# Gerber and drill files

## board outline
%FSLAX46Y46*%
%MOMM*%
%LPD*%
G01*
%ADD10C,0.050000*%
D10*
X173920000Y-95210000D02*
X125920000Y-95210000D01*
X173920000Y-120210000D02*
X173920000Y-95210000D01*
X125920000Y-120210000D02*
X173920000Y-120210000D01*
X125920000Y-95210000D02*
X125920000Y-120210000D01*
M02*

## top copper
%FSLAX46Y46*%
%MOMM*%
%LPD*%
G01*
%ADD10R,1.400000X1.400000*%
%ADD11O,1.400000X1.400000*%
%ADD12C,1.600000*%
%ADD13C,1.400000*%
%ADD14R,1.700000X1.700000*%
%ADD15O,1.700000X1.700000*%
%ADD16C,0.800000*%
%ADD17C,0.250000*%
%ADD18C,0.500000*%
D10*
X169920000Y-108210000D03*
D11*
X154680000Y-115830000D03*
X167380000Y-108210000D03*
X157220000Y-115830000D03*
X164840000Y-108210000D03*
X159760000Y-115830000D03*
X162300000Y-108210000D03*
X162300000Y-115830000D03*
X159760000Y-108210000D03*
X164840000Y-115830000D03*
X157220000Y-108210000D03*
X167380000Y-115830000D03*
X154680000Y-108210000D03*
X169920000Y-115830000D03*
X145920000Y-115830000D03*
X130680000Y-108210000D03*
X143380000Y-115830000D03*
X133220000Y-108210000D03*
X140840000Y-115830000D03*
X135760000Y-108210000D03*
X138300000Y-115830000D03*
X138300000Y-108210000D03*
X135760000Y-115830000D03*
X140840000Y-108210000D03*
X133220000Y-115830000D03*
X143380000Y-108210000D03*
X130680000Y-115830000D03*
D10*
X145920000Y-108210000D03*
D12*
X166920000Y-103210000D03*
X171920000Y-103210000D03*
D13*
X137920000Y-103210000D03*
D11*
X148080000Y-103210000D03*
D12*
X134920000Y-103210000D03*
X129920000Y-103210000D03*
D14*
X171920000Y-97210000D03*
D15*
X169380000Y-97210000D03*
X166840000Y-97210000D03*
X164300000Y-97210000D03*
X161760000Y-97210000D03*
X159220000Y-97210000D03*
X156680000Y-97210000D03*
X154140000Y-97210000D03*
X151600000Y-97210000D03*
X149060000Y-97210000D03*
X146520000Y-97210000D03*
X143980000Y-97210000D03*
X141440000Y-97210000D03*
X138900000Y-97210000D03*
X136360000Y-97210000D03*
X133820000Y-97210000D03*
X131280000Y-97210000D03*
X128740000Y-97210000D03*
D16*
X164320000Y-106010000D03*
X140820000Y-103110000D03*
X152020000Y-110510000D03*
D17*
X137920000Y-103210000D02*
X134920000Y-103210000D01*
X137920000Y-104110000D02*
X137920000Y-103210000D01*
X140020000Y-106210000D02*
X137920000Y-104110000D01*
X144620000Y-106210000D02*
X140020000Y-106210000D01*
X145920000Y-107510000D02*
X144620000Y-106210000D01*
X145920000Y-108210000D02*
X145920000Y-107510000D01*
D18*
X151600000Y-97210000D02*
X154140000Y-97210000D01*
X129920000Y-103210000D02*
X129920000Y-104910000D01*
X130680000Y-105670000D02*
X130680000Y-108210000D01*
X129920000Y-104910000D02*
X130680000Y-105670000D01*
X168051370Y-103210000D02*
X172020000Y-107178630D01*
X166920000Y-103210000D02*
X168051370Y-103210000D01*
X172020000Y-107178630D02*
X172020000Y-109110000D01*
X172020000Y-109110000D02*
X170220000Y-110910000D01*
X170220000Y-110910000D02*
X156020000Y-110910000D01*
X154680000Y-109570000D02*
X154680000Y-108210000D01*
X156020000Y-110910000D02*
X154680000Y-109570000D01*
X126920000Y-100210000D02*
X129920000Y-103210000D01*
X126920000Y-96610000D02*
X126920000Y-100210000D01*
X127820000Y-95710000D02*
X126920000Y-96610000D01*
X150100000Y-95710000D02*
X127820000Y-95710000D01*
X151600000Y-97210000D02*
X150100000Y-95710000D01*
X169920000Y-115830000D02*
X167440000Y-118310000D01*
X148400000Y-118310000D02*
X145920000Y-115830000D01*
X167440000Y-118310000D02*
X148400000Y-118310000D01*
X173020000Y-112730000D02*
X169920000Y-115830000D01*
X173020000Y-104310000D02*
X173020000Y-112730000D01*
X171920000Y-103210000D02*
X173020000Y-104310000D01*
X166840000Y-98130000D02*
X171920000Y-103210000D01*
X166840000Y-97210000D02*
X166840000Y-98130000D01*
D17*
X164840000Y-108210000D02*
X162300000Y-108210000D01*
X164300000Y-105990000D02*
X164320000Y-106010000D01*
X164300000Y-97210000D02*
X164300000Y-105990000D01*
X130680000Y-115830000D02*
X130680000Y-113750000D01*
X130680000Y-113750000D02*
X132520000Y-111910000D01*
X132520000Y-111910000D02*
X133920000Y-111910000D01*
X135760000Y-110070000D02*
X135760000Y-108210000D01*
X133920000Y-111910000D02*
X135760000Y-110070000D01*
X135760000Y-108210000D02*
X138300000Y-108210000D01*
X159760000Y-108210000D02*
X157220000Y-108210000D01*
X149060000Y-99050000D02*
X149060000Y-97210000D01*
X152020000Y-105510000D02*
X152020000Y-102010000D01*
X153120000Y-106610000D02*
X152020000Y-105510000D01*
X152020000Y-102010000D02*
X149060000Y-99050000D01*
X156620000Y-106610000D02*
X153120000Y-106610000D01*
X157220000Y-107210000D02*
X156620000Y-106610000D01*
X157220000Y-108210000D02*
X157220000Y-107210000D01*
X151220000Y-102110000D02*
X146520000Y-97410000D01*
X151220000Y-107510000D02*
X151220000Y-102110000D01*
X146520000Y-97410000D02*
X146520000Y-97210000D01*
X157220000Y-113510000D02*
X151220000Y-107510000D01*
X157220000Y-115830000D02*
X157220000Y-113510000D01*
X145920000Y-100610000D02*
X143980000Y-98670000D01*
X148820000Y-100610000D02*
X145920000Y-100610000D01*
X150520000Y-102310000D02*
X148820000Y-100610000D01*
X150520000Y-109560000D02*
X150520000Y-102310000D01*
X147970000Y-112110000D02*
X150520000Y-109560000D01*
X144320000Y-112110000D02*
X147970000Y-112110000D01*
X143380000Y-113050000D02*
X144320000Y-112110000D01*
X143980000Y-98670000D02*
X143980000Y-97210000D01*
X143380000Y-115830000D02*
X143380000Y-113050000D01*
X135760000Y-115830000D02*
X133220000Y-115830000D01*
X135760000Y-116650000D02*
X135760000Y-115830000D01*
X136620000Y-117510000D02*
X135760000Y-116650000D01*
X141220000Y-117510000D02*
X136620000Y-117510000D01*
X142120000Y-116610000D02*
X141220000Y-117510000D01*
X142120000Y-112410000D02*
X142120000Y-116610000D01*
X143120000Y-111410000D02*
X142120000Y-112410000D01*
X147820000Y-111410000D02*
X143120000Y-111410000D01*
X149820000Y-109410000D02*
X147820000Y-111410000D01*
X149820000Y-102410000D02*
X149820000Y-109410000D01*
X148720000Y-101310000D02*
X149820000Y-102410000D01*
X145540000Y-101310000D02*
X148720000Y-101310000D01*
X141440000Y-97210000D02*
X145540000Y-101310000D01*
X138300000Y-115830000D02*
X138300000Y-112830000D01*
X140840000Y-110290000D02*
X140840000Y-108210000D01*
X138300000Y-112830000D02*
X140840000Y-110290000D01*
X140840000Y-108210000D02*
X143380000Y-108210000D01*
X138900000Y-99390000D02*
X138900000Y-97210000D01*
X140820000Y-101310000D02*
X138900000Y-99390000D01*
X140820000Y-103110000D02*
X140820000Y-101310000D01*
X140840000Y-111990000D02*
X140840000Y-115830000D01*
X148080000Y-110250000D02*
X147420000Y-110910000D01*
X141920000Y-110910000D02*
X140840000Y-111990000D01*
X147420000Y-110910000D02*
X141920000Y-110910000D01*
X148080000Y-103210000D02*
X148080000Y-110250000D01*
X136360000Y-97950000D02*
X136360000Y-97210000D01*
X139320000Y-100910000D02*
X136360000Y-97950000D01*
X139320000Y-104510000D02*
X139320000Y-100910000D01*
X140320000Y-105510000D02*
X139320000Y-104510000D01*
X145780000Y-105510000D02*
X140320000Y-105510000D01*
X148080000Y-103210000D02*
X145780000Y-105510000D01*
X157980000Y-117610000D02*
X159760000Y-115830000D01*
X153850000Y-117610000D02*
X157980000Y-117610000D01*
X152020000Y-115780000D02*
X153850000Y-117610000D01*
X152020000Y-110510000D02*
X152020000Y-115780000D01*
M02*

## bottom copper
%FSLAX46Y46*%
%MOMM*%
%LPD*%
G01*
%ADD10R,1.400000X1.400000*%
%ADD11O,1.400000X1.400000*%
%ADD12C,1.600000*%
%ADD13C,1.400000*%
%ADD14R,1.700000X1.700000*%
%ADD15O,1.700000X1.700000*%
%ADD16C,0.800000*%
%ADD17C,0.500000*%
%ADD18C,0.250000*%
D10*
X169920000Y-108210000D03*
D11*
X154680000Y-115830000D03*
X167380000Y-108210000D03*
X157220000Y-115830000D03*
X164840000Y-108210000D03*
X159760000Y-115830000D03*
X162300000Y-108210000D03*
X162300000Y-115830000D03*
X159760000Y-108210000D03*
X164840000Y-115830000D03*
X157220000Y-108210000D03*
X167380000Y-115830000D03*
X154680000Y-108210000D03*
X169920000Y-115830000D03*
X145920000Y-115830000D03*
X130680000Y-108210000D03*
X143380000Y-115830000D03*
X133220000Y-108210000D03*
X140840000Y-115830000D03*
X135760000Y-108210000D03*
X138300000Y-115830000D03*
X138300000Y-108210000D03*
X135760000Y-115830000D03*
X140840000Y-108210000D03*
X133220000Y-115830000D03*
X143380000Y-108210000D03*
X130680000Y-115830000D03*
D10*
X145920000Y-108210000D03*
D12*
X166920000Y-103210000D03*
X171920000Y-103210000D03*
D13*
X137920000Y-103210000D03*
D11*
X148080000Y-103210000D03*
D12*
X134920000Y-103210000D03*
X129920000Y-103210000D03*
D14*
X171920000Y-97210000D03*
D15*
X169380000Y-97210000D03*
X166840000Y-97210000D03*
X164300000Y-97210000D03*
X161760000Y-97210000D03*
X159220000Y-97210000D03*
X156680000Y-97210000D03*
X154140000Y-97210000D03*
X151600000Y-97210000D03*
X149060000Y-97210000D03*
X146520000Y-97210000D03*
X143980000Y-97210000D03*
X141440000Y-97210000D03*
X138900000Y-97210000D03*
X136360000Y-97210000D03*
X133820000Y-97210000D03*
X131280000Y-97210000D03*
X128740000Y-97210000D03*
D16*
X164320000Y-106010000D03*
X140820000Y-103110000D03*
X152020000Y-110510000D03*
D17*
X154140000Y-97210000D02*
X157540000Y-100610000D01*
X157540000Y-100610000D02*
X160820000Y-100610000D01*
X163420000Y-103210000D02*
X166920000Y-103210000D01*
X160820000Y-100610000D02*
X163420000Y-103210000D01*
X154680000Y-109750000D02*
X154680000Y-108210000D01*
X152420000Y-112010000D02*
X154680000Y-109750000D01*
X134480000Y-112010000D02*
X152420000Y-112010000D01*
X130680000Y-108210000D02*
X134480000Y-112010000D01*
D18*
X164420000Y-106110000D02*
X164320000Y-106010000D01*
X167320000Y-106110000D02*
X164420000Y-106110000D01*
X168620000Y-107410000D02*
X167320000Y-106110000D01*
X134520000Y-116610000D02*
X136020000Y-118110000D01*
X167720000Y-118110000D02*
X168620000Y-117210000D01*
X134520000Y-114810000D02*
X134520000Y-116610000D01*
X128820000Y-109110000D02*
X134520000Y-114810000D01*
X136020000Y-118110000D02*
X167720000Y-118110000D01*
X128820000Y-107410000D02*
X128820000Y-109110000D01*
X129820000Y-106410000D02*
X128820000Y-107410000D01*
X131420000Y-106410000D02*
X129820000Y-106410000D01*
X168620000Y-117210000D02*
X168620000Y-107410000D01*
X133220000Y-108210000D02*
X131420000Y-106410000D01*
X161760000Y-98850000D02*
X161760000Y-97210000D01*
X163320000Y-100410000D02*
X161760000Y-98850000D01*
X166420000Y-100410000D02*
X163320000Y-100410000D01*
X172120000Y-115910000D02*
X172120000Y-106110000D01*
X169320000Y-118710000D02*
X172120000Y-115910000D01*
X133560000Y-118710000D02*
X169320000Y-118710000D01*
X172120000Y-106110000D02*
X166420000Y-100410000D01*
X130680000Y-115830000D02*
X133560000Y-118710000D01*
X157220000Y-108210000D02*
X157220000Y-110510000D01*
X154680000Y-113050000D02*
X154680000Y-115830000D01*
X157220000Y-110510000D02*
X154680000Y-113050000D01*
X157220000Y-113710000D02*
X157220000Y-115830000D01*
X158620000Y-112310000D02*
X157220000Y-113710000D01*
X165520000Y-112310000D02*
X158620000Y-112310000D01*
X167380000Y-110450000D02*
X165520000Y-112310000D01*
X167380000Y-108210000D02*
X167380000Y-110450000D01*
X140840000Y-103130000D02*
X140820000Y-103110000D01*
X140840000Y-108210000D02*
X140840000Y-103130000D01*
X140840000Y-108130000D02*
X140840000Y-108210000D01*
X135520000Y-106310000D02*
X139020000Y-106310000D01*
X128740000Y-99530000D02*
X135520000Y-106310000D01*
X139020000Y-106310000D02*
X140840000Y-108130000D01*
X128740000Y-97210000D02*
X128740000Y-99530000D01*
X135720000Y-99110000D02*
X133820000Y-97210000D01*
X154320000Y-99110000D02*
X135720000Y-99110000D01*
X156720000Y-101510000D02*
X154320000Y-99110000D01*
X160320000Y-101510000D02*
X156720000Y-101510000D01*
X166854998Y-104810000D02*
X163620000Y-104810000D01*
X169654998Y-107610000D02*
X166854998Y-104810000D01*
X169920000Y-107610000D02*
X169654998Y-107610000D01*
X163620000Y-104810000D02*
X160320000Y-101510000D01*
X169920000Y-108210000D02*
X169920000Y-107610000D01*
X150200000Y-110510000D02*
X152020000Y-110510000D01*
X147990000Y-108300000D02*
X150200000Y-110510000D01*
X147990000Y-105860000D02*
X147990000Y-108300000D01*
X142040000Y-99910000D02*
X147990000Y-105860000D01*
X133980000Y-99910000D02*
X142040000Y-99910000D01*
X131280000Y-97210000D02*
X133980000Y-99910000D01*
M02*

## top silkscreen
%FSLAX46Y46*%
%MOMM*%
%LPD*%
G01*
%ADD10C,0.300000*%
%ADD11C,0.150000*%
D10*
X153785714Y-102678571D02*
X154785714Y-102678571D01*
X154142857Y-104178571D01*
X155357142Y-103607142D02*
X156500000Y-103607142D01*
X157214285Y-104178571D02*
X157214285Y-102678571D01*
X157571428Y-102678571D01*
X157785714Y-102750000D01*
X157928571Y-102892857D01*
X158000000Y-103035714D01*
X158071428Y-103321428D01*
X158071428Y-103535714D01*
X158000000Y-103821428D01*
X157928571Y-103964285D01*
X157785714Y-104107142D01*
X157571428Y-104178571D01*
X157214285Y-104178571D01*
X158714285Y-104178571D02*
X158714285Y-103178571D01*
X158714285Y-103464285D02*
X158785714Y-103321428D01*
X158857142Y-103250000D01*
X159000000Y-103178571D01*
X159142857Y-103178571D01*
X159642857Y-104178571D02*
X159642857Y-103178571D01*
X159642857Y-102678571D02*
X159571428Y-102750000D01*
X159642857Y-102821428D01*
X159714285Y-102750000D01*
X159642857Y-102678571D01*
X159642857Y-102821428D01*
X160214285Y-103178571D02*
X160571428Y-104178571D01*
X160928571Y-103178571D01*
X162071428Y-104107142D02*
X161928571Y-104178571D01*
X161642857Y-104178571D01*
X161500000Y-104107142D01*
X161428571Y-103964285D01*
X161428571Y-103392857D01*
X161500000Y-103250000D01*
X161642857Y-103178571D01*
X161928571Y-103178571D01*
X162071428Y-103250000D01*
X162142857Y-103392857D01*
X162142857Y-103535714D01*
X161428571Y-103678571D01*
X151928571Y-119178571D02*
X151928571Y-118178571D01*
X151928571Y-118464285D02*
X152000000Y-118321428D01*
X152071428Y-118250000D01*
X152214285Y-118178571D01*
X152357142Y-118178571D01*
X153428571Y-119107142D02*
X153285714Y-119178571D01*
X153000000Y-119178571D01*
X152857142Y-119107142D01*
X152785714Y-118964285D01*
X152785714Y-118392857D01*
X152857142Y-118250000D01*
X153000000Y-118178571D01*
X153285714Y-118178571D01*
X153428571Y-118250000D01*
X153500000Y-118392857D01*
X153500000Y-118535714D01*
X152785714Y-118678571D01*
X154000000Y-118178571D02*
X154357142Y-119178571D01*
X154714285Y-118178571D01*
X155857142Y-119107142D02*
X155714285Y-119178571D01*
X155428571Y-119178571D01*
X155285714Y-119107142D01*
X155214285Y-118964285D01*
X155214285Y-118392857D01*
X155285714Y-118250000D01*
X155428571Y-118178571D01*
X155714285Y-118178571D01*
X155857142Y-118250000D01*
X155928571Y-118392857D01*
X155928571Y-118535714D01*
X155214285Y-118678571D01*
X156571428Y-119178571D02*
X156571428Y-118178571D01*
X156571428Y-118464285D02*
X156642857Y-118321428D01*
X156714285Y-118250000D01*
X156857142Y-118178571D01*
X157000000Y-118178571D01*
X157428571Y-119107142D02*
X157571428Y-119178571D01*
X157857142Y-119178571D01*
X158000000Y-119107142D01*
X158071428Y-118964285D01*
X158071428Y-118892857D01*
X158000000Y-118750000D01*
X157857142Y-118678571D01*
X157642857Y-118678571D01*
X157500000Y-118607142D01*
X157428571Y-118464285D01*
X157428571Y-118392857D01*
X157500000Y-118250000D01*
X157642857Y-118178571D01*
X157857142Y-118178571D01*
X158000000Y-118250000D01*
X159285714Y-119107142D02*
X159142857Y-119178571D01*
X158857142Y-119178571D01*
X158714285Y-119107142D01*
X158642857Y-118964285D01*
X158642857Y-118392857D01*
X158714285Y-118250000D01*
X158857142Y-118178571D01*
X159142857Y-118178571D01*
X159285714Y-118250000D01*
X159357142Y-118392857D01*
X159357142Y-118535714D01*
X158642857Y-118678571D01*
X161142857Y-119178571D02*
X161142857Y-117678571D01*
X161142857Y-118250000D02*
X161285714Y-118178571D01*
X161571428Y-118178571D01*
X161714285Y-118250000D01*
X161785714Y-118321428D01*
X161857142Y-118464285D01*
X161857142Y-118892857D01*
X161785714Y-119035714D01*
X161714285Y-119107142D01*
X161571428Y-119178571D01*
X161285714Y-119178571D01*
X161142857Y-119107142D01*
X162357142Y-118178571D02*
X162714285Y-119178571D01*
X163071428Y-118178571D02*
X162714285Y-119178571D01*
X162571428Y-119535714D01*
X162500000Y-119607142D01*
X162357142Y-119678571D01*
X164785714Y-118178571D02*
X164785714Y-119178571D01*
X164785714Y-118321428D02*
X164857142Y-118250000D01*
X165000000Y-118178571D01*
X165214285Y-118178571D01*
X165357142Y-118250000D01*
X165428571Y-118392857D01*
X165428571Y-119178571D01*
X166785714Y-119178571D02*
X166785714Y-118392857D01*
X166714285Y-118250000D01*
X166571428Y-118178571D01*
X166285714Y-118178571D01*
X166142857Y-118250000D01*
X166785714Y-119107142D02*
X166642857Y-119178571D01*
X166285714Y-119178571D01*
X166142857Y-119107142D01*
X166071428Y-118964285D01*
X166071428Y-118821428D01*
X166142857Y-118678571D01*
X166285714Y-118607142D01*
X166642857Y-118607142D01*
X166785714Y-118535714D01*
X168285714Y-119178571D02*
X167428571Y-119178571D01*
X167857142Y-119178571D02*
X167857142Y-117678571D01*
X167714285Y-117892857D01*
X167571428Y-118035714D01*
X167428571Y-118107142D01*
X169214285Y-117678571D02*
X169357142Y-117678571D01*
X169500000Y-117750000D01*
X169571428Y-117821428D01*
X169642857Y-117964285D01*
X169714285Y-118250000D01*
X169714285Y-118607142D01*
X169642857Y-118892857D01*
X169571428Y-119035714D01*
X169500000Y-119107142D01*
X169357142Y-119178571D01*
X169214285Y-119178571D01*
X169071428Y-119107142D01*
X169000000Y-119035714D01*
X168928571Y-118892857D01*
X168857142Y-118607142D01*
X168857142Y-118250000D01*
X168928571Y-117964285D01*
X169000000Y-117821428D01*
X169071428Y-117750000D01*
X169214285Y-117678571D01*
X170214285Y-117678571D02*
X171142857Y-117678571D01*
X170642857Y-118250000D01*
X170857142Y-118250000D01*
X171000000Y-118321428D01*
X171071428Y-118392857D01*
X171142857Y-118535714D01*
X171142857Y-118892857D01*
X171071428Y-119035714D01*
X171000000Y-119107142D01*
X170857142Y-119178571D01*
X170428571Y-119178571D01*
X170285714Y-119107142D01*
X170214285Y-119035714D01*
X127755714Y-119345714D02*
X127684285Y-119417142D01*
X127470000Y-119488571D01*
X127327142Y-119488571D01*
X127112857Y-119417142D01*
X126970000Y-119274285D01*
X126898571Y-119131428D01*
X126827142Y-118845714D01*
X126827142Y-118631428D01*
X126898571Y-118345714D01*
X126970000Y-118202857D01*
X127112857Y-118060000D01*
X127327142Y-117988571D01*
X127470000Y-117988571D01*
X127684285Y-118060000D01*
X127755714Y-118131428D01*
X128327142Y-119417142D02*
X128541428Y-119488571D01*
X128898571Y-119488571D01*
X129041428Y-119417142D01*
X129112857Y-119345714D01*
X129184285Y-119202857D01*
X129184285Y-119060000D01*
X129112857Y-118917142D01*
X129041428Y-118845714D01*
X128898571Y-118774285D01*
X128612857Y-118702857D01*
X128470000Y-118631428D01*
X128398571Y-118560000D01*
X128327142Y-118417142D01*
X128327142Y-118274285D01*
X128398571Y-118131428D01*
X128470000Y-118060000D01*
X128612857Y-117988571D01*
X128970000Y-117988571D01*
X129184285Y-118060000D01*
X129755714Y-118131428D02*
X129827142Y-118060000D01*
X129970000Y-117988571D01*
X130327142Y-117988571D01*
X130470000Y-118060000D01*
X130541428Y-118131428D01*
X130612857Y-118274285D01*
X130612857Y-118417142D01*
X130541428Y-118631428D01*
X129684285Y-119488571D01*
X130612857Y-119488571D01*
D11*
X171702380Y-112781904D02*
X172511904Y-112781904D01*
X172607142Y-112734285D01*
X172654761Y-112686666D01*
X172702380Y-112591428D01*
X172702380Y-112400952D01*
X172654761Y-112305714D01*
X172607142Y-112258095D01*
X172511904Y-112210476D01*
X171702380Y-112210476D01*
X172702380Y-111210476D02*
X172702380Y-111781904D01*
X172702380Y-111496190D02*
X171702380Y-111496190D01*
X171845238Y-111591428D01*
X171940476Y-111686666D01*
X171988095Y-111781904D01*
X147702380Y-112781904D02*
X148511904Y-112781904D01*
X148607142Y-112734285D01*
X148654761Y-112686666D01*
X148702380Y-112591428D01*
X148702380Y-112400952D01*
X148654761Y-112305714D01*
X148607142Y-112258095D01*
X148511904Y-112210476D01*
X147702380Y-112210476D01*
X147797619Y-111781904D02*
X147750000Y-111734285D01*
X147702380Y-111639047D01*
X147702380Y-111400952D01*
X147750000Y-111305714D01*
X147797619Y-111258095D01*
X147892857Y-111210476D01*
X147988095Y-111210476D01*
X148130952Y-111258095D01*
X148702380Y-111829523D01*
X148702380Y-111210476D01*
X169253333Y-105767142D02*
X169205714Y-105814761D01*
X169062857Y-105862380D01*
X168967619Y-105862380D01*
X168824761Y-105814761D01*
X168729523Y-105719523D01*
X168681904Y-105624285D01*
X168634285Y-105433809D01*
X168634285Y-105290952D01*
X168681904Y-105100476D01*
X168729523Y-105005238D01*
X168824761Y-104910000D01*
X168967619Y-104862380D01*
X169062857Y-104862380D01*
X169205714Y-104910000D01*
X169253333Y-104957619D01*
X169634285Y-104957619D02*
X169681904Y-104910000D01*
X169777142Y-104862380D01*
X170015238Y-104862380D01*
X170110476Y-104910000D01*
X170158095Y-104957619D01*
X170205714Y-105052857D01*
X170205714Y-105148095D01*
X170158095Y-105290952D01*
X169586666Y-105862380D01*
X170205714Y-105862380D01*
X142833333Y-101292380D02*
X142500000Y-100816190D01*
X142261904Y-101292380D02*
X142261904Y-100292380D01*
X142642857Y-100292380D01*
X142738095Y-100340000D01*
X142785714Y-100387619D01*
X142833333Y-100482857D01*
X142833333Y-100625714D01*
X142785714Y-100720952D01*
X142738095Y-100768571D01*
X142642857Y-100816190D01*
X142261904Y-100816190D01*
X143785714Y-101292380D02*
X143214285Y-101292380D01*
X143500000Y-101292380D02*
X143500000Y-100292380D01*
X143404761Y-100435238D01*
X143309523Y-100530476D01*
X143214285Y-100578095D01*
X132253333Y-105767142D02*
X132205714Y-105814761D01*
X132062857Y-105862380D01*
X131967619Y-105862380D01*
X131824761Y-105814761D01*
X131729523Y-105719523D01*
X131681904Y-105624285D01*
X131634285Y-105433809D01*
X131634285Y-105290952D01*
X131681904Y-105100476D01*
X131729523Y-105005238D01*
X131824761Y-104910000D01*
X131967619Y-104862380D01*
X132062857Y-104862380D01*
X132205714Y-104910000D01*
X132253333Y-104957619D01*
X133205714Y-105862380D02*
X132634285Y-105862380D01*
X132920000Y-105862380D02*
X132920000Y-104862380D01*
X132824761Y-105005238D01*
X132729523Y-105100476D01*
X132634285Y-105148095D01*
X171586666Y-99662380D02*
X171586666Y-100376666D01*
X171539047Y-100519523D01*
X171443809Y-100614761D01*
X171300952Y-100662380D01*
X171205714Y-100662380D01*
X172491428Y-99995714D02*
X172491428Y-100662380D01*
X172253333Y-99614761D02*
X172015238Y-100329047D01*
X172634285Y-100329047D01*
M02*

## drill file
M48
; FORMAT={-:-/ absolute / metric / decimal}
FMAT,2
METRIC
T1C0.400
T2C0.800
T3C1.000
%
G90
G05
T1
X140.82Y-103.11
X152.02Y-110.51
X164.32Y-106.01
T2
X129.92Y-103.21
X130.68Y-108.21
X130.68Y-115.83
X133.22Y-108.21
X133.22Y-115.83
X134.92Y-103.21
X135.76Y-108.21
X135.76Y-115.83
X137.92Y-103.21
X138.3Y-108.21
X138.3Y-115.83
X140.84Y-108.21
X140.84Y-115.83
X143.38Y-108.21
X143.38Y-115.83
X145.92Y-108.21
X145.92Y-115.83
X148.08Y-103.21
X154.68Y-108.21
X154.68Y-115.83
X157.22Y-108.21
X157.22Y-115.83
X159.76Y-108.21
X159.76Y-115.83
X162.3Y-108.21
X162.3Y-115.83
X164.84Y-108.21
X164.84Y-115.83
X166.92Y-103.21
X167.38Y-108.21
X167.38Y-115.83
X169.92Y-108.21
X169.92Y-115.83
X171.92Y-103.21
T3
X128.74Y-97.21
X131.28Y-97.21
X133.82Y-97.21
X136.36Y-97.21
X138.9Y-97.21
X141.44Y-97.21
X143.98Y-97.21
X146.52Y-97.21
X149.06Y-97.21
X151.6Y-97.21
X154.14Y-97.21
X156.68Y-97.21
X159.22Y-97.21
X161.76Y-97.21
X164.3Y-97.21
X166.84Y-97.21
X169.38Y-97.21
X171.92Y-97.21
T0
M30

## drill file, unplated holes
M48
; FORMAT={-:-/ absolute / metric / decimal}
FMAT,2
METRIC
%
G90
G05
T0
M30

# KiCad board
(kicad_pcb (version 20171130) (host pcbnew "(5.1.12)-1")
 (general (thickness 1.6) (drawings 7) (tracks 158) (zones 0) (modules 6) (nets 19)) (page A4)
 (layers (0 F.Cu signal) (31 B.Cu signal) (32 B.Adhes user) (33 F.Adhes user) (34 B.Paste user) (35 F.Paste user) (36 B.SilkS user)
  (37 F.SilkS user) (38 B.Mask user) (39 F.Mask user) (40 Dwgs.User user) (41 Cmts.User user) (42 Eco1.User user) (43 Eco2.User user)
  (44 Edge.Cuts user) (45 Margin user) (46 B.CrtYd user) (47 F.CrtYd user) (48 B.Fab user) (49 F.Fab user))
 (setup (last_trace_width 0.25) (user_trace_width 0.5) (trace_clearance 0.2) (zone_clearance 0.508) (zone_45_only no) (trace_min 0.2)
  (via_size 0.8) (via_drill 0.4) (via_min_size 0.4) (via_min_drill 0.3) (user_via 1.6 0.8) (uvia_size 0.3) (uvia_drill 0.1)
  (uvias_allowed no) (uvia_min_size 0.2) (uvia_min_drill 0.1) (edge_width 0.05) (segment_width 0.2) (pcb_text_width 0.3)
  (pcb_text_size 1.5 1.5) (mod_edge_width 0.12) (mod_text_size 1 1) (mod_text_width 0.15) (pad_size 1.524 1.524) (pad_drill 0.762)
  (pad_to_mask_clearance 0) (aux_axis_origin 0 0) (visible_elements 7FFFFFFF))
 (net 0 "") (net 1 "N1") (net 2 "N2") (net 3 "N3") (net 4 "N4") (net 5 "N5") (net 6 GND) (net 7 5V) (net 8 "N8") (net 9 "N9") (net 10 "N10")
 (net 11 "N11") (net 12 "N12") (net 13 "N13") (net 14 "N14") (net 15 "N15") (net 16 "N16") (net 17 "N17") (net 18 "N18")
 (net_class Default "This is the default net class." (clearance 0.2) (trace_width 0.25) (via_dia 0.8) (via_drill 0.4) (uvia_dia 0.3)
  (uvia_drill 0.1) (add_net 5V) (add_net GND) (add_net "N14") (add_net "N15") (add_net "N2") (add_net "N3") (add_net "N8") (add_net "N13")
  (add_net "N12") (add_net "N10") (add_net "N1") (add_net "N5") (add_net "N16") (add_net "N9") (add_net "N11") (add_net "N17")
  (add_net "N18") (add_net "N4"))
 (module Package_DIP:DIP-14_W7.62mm (layer F.Cu) (at 169.92 108.21 270)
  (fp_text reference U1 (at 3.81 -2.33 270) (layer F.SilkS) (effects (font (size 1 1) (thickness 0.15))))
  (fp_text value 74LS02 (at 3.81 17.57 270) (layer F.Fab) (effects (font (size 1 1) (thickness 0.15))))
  (pad 1 thru_hole rect (at 0 0 270) (size 1.4 1.4) (drill 0.8) (layers *.Cu *.Mask) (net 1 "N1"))
  (pad 8 thru_hole oval (at 7.62 15.24 270) (size 1.4 1.4) (drill 0.8) (layers *.Cu *.Mask) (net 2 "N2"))
  (pad 2 thru_hole oval (at 0 2.54 270) (size 1.4 1.4) (drill 0.8) (layers *.Cu *.Mask) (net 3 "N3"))
  (pad 9 thru_hole oval (at 7.62 12.7 270) (size 1.4 1.4) (drill 0.8) (layers *.Cu *.Mask) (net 3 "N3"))
  (pad 3 thru_hole oval (at 0 5.08 270) (size 1.4 1.4) (drill 0.8) (layers *.Cu *.Mask) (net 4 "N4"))
  (pad 10 thru_hole oval (at 7.62 10.16 270) (size 1.4 1.4) (drill 0.8) (layers *.Cu *.Mask) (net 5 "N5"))
  (pad 4 thru_hole oval (at 0 7.62 270) (size 1.4 1.4) (drill 0.8) (layers *.Cu *.Mask) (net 4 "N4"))
  (pad 11 thru_hole oval (at 7.62 7.62 270) (size 1.4 1.4) (drill 0.8) (layers *.Cu *.Mask))
  (pad 5 thru_hole oval (at 0 10.16 270) (size 1.4 1.4) (drill 0.8) (layers *.Cu *.Mask) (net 2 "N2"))
  (pad 12 thru_hole oval (at 7.62 5.08 270) (size 1.4 1.4) (drill 0.8) (layers *.Cu *.Mask))
  (pad 6 thru_hole oval (at 0 12.7 270) (size 1.4 1.4) (drill 0.8) (layers *.Cu *.Mask) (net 2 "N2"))
  (pad 13 thru_hole oval (at 7.62 2.54 270) (size 1.4 1.4) (drill 0.8) (layers *.Cu *.Mask))
  (pad 7 thru_hole oval (at 0 15.24 270) (size 1.4 1.4) (drill 0.8) (layers *.Cu *.Mask) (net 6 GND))
  (pad 14 thru_hole oval (at 7.62 0 270) (size 1.4 1.4) (drill 0.8) (layers *.Cu *.Mask) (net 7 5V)))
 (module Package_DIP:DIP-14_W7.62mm (layer F.Cu) (at 145.92 108.21 270)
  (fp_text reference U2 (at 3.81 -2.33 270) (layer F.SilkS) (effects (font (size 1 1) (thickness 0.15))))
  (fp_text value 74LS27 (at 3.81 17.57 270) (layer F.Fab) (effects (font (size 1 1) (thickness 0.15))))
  (pad 14 thru_hole oval (at 7.62 0 270) (size 1.4 1.4) (drill 0.8) (layers *.Cu *.Mask) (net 7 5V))
  (pad 7 thru_hole oval (at 0 15.24 270) (size 1.4 1.4) (drill 0.8) (layers *.Cu *.Mask) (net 6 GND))
  (pad 13 thru_hole oval (at 7.62 2.54 270) (size 1.4 1.4) (drill 0.8) (layers *.Cu *.Mask) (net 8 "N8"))
  (pad 6 thru_hole oval (at 0 12.7 270) (size 1.4 1.4) (drill 0.8) (layers *.Cu *.Mask) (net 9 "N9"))
  (pad 12 thru_hole oval (at 7.62 5.08 270) (size 1.4 1.4) (drill 0.8) (layers *.Cu *.Mask) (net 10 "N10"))
  (pad 5 thru_hole oval (at 0 10.16 270) (size 1.4 1.4) (drill 0.8) (layers *.Cu *.Mask) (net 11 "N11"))
  (pad 11 thru_hole oval (at 7.62 7.62 270) (size 1.4 1.4) (drill 0.8) (layers *.Cu *.Mask) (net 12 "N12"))
  (pad 4 thru_hole oval (at 0 7.62 270) (size 1.4 1.4) (drill 0.8) (layers *.Cu *.Mask) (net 11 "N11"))
  (pad 10 thru_hole oval (at 7.62 10.16 270) (size 1.4 1.4) (drill 0.8) (layers *.Cu *.Mask) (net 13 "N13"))
  (pad 3 thru_hole oval (at 0 5.08 270) (size 1.4 1.4) (drill 0.8) (layers *.Cu *.Mask) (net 12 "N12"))
  (pad 9 thru_hole oval (at 7.62 12.7 270) (size 1.4 1.4) (drill 0.8) (layers *.Cu *.Mask) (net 13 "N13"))
  (pad 2 thru_hole oval (at 0 2.54 270) (size 1.4 1.4) (drill 0.8) (layers *.Cu *.Mask) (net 12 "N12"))
  (pad 8 thru_hole oval (at 7.62 15.24 270) (size 1.4 1.4) (drill 0.8) (layers *.Cu *.Mask) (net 11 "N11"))
  (pad 1 thru_hole rect (at 0 0 270) (size 1.4 1.4) (drill 0.8) (layers *.Cu *.Mask) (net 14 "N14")))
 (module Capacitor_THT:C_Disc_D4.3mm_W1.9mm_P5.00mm (layer F.Cu) (at 171.92 103.21 180)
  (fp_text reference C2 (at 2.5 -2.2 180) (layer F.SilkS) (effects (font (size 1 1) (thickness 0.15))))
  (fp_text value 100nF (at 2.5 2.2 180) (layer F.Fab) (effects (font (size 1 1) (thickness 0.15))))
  (pad 2 thru_hole circle (at 5 0 180) (size 1.6 1.6) (drill 0.8) (layers *.Cu *.Mask) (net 6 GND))
  (pad 1 thru_hole circle (at 0 0 180) (size 1.6 1.6) (drill 0.8) (layers *.Cu *.Mask) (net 7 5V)))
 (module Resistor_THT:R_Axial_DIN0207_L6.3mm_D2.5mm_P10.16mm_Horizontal (layer F.Cu) (at 137.92 103.21)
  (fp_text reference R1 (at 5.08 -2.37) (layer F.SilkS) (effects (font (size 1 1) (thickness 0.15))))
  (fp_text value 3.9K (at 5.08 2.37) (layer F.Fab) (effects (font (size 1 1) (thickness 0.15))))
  (pad 1 thru_hole circle (at 0 0) (size 1.4 1.4) (drill 0.8) (layers *.Cu *.Mask) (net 14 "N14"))
  (pad 2 thru_hole oval (at 10.16 0) (size 1.4 1.4) (drill 0.8) (layers *.Cu *.Mask) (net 10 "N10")))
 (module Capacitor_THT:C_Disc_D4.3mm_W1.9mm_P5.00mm (layer F.Cu) (at 134.92 103.21 180)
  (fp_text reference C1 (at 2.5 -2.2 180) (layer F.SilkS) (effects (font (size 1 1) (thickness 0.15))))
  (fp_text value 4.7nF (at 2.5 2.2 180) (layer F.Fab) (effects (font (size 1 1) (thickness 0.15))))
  (pad 1 thru_hole circle (at 0 0 180) (size 1.6 1.6) (drill 0.8) (layers *.Cu *.Mask) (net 14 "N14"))
  (pad 2 thru_hole circle (at 5 0 180) (size 1.6 1.6) (drill 0.8) (layers *.Cu *.Mask) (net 6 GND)))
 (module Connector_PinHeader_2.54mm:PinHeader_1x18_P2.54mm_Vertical (layer F.Cu) (at 171.92 97.21 270)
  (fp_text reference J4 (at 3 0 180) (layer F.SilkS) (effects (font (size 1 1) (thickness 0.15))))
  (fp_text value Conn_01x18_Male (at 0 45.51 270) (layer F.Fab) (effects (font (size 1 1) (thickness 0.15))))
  (pad 1 thru_hole rect (at 0 0 270) (size 1.7 1.7) (drill 1) (layers *.Cu *.Mask) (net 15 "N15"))
  (pad 2 thru_hole oval (at 0 2.54 270) (size 1.7 1.7) (drill 1) (layers *.Cu *.Mask) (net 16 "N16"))
  (pad 3 thru_hole oval (at 0 5.08 270) (size 1.7 1.7) (drill 1) (layers *.Cu *.Mask) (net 7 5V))
  (pad 4 thru_hole oval (at 0 7.62 270) (size 1.7 1.7) (drill 1) (layers *.Cu *.Mask) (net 9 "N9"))
  (pad 5 thru_hole oval (at 0 10.16 270) (size 1.7 1.7) (drill 1) (layers *.Cu *.Mask) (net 11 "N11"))
  (pad 6 thru_hole oval (at 0 12.7 270) (size 1.7 1.7) (drill 1) (layers *.Cu *.Mask) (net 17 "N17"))
  (pad 7 thru_hole oval (at 0 15.24 270) (size 1.7 1.7) (drill 1) (layers *.Cu *.Mask) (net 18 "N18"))
  (pad 8 thru_hole oval (at 0 17.78 270) (size 1.7 1.7) (drill 1) (layers *.Cu *.Mask) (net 6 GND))
  (pad 9 thru_hole oval (at 0 20.32 270) (size 1.7 1.7) (drill 1) (layers *.Cu *.Mask) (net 6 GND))
  (pad 10 thru_hole oval (at 0 22.86 270) (size 1.7 1.7) (drill 1) (layers *.Cu *.Mask) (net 2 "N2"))
  (pad 11 thru_hole oval (at 0 25.4 270) (size 1.7 1.7) (drill 1) (layers *.Cu *.Mask) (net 3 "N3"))
  (pad 12 thru_hole oval (at 0 27.94 270) (size 1.7 1.7) (drill 1) (layers *.Cu *.Mask) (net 8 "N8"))
  (pad 13 thru_hole oval (at 0 30.48 270) (size 1.7 1.7) (drill 1) (layers *.Cu *.Mask) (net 13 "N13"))
  (pad 14 thru_hole oval (at 0 33.02 270) (size 1.7 1.7) (drill 1) (layers *.Cu *.Mask) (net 12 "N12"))
  (pad 15 thru_hole oval (at 0 35.56 270) (size 1.7 1.7) (drill 1) (layers *.Cu *.Mask) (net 10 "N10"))
  (pad 16 thru_hole oval (at 0 38.1 270) (size 1.7 1.7) (drill 1) (layers *.Cu *.Mask) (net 1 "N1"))
  (pad 17 thru_hole oval (at 0 40.64 270) (size 1.7 1.7) (drill 1) (layers *.Cu *.Mask) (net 5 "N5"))
  (pad 18 thru_hole oval (at 0 43.18 270) (size 1.7 1.7) (drill 1) (layers *.Cu *.Mask) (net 12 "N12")))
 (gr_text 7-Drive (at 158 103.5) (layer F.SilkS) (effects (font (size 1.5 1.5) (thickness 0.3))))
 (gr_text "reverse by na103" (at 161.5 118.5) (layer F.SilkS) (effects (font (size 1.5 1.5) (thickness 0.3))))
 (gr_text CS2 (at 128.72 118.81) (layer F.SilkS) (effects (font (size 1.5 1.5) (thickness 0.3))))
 (gr_line (start 173.92 95.21) (end 125.92 95.21) (layer Edge.Cuts) (width 0.05))
 (gr_line (start 173.92 120.21) (end 173.92 95.21) (layer Edge.Cuts) (width 0.05))
 (gr_line (start 125.92 120.21) (end 173.92 120.21) (layer Edge.Cuts) (width 0.05))
 (gr_line (start 125.92 95.21) (end 125.92 120.21) (layer Edge.Cuts) (width 0.05))
 (segment (start 137.92 103.21) (end 134.92 103.21) (width 0.25) (layer F.Cu) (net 14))
 (segment (start 137.92 104.11) (end 137.92 103.21) (width 0.25) (layer F.Cu) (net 14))
 (segment (start 140.02 106.21) (end 137.92 104.11) (width 0.25) (layer F.Cu) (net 14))
 (segment (start 144.62 106.21) (end 140.02 106.21) (width 0.25) (layer F.Cu) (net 14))
 (segment (start 145.92 107.51) (end 144.62 106.21) (width 0.25) (layer F.Cu) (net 14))
 (segment (start 145.92 108.21) (end 145.92 107.51) (width 0.25) (layer F.Cu) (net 14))
 (segment (start 151.6 97.21) (end 154.14 97.21) (width 0.5) (layer F.Cu) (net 6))
 (segment (start 129.92 103.21) (end 129.92 104.91) (width 0.5) (layer F.Cu) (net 6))
 (segment (start 130.68 105.67) (end 130.68 108.21) (width 0.5) (layer F.Cu) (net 6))
 (segment (start 129.92 104.91) (end 130.68 105.67) (width 0.5) (layer F.Cu) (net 6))
 (segment (start 154.14 97.21) (end 157.54 100.61) (width 0.5) (layer B.Cu) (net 6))
 (segment (start 157.54 100.61) (end 160.82 100.61) (width 0.5) (layer B.Cu) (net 6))
 (segment (start 163.42 103.21) (end 166.92 103.21) (width 0.5) (layer B.Cu) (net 6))
 (segment (start 160.82 100.61) (end 163.42 103.21) (width 0.5) (layer B.Cu) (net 6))
 (segment (start 168.05137 103.21) (end 172.02 107.17863) (width 0.5) (layer F.Cu) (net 6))
 (segment (start 166.92 103.21) (end 168.05137 103.21) (width 0.5) (layer F.Cu) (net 6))
 (segment (start 172.02 107.17863) (end 172.02 109.11) (width 0.5) (layer F.Cu) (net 6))
 (segment (start 172.02 109.11) (end 170.22 110.91) (width 0.5) (layer F.Cu) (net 6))
 (segment (start 170.22 110.91) (end 156.02 110.91) (width 0.5) (layer F.Cu) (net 6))
 (segment (start 154.68 109.57) (end 154.68 108.21) (width 0.5) (layer F.Cu) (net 6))
 (segment (start 156.02 110.91) (end 154.68 109.57) (width 0.5) (layer F.Cu) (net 6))
 (segment (start 154.68 109.75) (end 154.68 108.21) (width 0.5) (layer B.Cu) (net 6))
 (segment (start 152.42 112.01) (end 154.68 109.75) (width 0.5) (layer B.Cu) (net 6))
 (segment (start 134.48 112.01) (end 152.42 112.01) (width 0.5) (layer B.Cu) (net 6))
 (segment (start 130.68 108.21) (end 134.48 112.01) (width 0.5) (layer B.Cu) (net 6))
 (segment (start 126.92 100.21) (end 129.92 103.21) (width 0.5) (layer F.Cu) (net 6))
 (segment (start 126.92 96.61) (end 126.92 100.21) (width 0.5) (layer F.Cu) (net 6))
 (segment (start 127.82 95.71) (end 126.92 96.61) (width 0.5) (layer F.Cu) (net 6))
 (segment (start 150.1 95.71) (end 127.82 95.71) (width 0.5) (layer F.Cu) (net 6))
 (segment (start 151.6 97.21) (end 150.1 95.71) (width 0.5) (layer F.Cu) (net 6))
 (segment (start 169.92 115.83) (end 167.44 118.31) (width 0.5) (layer F.Cu) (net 7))
 (segment (start 148.4 118.31) (end 145.92 115.83) (width 0.5) (layer F.Cu) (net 7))
 (segment (start 167.44 118.31) (end 148.4 118.31) (width 0.5) (layer F.Cu) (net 7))
 (segment (start 173.02 112.73) (end 169.92 115.83) (width 0.5) (layer F.Cu) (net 7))
 (segment (start 173.02 104.31) (end 173.02 112.73) (width 0.5) (layer F.Cu) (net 7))
 (segment (start 171.92 103.21) (end 173.02 104.31) (width 0.5) (layer F.Cu) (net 7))
 (segment (start 166.84 98.13) (end 171.92 103.21) (width 0.5) (layer F.Cu) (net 7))
 (segment (start 166.84 97.21) (end 166.84 98.13) (width 0.5) (layer F.Cu) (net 7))
 (segment (start 164.84 108.21) (end 162.3 108.21) (width 0.25) (layer F.Cu) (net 4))
 (via (at 164.32 106.01) (size 0.8) (drill 0.4) (layers F.Cu B.Cu) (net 9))
 (segment (start 164.3 105.99) (end 164.32 106.01) (width 0.25) (layer F.Cu) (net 9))
 (segment (start 164.3 97.21) (end 164.3 105.99) (width 0.25) (layer F.Cu) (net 9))
 (segment (start 164.42 106.11) (end 164.32 106.01) (width 0.25) (layer B.Cu) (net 9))
 (segment (start 167.32 106.11) (end 164.42 106.11) (width 0.25) (layer B.Cu) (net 9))
 (segment (start 168.62 107.41) (end 167.32 106.11) (width 0.25) (layer B.Cu) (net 9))
 (segment (start 134.52 116.61) (end 136.02 118.11) (width 0.25) (layer B.Cu) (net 9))
 (segment (start 167.72 118.11) (end 168.62 117.21) (width 0.25) (layer B.Cu) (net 9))
 (segment (start 134.52 114.81) (end 134.52 116.61) (width 0.25) (layer B.Cu) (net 9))
 (segment (start 128.82 109.11) (end 134.52 114.81) (width 0.25) (layer B.Cu) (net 9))
 (segment (start 136.02 118.11) (end 167.72 118.11) (width 0.25) (layer B.Cu) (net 9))
 (segment (start 128.82 107.41) (end 128.82 109.11) (width 0.25) (layer B.Cu) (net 9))
 (segment (start 129.82 106.41) (end 128.82 107.41) (width 0.25) (layer B.Cu) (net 9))
 (segment (start 131.42 106.41) (end 129.82 106.41) (width 0.25) (layer B.Cu) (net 9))
 (segment (start 168.62 117.21) (end 168.62 107.41) (width 0.25) (layer B.Cu) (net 9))
 (segment (start 133.22 108.21) (end 131.42 106.41) (width 0.25) (layer B.Cu) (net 9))
 (segment (start 130.68 115.83) (end 130.68 113.75) (width 0.25) (layer F.Cu) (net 11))
 (segment (start 130.68 113.75) (end 132.52 111.91) (width 0.25) (layer F.Cu) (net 11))
 (segment (start 132.52 111.91) (end 133.92 111.91) (width 0.25) (layer F.Cu) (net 11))
 (segment (start 135.76 110.07) (end 135.76 108.21) (width 0.25) (layer F.Cu) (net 11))
 (segment (start 133.92 111.91) (end 135.76 110.07) (width 0.25) (layer F.Cu) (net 11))
 (segment (start 135.76 108.21) (end 138.3 108.21) (width 0.25) (layer F.Cu) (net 11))
 (segment (start 161.76 98.85) (end 161.76 97.21) (width 0.25) (layer B.Cu) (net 11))
 (segment (start 163.32 100.41) (end 161.76 98.85) (width 0.25) (layer B.Cu) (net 11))
 (segment (start 166.42 100.41) (end 163.32 100.41) (width 0.25) (layer B.Cu) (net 11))
 (segment (start 172.12 115.91) (end 172.12 106.11) (width 0.25) (layer B.Cu) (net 11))
 (segment (start 169.32 118.71) (end 172.12 115.91) (width 0.25) (layer B.Cu) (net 11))
 (segment (start 133.56 118.71) (end 169.32 118.71) (width 0.25) (layer B.Cu) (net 11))
 (segment (start 172.12 106.11) (end 166.42 100.41) (width 0.25) (layer B.Cu) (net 11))
 (segment (start 130.68 115.83) (end 133.56 118.71) (width 0.25) (layer B.Cu) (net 11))
 (segment (start 157.22 108.21) (end 157.22 110.51) (width 0.25) (layer B.Cu) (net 2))
 (segment (start 154.68 113.05) (end 154.68 115.83) (width 0.25) (layer B.Cu) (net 2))
 (segment (start 157.22 110.51) (end 154.68 113.05) (width 0.25) (layer B.Cu) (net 2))
 (segment (start 159.76 108.21) (end 157.22 108.21) (width 0.25) (layer F.Cu) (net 2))
 (segment (start 149.06 99.05) (end 149.06 97.21) (width 0.25) (layer F.Cu) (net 2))
 (segment (start 152.02 105.51) (end 152.02 102.01) (width 0.25) (layer F.Cu) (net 2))
 (segment (start 153.12 106.61) (end 152.02 105.51) (width 0.25) (layer F.Cu) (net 2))
 (segment (start 152.02 102.01) (end 149.06 99.05) (width 0.25) (layer F.Cu) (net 2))
 (segment (start 156.62 106.61) (end 153.12 106.61) (width 0.25) (layer F.Cu) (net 2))
 (segment (start 157.22 107.21) (end 156.62 106.61) (width 0.25) (layer F.Cu) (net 2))
 (segment (start 157.22 108.21) (end 157.22 107.21) (width 0.25) (layer F.Cu) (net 2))
 (segment (start 157.22 113.71) (end 157.22 115.83) (width 0.25) (layer B.Cu) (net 3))
 (segment (start 158.62 112.31) (end 157.22 113.71) (width 0.25) (layer B.Cu) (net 3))
 (segment (start 165.52 112.31) (end 158.62 112.31) (width 0.25) (layer B.Cu) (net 3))
 (segment (start 167.38 110.45) (end 165.52 112.31) (width 0.25) (layer B.Cu) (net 3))
 (segment (start 167.38 108.21) (end 167.38 110.45) (width 0.25) (layer B.Cu) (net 3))
 (segment (start 151.22 102.11) (end 146.52 97.41) (width 0.25) (layer F.Cu) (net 3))
 (segment (start 151.22 107.51) (end 151.22 102.11) (width 0.25) (layer F.Cu) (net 3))
 (segment (start 146.52 97.41) (end 146.52 97.21) (width 0.25) (layer F.Cu) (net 3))
 (segment (start 157.22 113.51) (end 151.22 107.51) (width 0.25) (layer F.Cu) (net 3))
 (segment (start 157.22 115.83) (end 157.22 113.51) (width 0.25) (layer F.Cu) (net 3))
 (segment (start 145.92 100.61) (end 143.98 98.67) (width 0.25) (layer F.Cu) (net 8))
 (segment (start 148.82 100.61) (end 145.92 100.61) (width 0.25) (layer F.Cu) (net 8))
 (segment (start 150.52 102.31) (end 148.82 100.61) (width 0.25) (layer F.Cu) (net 8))
 (segment (start 150.52 109.56) (end 150.52 102.31) (width 0.25) (layer F.Cu) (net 8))
 (segment (start 147.97 112.11) (end 150.52 109.56) (width 0.25) (layer F.Cu) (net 8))
 (segment (start 144.32 112.11) (end 147.97 112.11) (width 0.25) (layer F.Cu) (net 8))
 (segment (start 143.38 113.05) (end 144.32 112.11) (width 0.25) (layer F.Cu) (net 8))
 (segment (start 143.98 98.67) (end 143.98 97.21) (width 0.25) (layer F.Cu) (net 8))
 (segment (start 143.38 115.83) (end 143.38 113.05) (width 0.25) (layer F.Cu) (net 8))
 (segment (start 135.76 115.83) (end 133.22 115.83) (width 0.25) (layer F.Cu) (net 13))
 (segment (start 135.76 116.65) (end 135.76 115.83) (width 0.25) (layer F.Cu) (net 13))
 (segment (start 136.62 117.51) (end 135.76 116.65) (width 0.25) (layer F.Cu) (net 13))
 (segment (start 141.22 117.51) (end 136.62 117.51) (width 0.25) (layer F.Cu) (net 13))
 (segment (start 142.12 116.61) (end 141.22 117.51) (width 0.25) (layer F.Cu) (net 13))
 (segment (start 142.12 112.41) (end 142.12 116.61) (width 0.25) (layer F.Cu) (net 13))
 (segment (start 143.12 111.41) (end 142.12 112.41) (width 0.25) (layer F.Cu) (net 13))
 (segment (start 147.82 111.41) (end 143.12 111.41) (width 0.25) (layer F.Cu) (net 13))
 (segment (start 149.82 109.41) (end 147.82 111.41) (width 0.25) (layer F.Cu) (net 13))
 (segment (start 149.82 102.41) (end 149.82 109.41) (width 0.25) (layer F.Cu) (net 13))
 (segment (start 148.72 101.31) (end 149.82 102.41) (width 0.25) (layer F.Cu) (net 13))
 (segment (start 145.54 101.31) (end 148.72 101.31) (width 0.25) (layer F.Cu) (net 13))
 (segment (start 141.44 97.21) (end 145.54 101.31) (width 0.25) (layer F.Cu) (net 13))
 (via (at 140.82 103.11) (size 0.8) (drill 0.4) (layers F.Cu B.Cu) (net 12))
 (segment (start 140.84 103.13) (end 140.82 103.11) (width 0.25) (layer B.Cu) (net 12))
 (segment (start 140.84 108.21) (end 140.84 103.13) (width 0.25) (layer B.Cu) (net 12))
 (segment (start 138.3 115.83) (end 138.3 112.83) (width 0.25) (layer F.Cu) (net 12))
 (segment (start 140.84 110.29) (end 140.84 108.21) (width 0.25) (layer F.Cu) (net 12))
 (segment (start 138.3 112.83) (end 140.84 110.29) (width 0.25) (layer F.Cu) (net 12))
 (segment (start 140.84 108.21) (end 143.38 108.21) (width 0.25) (layer F.Cu) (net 12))
 (segment (start 138.9 99.39) (end 138.9 97.21) (width 0.25) (layer F.Cu) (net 12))
 (segment (start 140.82 101.31) (end 138.9 99.39) (width 0.25) (layer F.Cu) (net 12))
 (segment (start 140.82 103.11) (end 140.82 101.31) (width 0.25) (layer F.Cu) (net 12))
 (segment (start 140.84 108.13) (end 140.84 108.21) (width 0.25) (layer B.Cu) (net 12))
 (segment (start 135.52 106.31) (end 139.02 106.31) (width 0.25) (layer B.Cu) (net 12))
 (segment (start 128.74 99.53) (end 135.52 106.31) (width 0.25) (layer B.Cu) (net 12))
 (segment (start 139.02 106.31) (end 140.84 108.13) (width 0.25) (layer B.Cu) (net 12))
 (segment (start 128.74 97.21) (end 128.74 99.53) (width 0.25) (layer B.Cu) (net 12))
 (segment (start 140.84 111.99) (end 140.84 115.83) (width 0.25) (layer F.Cu) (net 10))
 (segment (start 148.08 110.25) (end 147.42 110.91) (width 0.25) (layer F.Cu) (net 10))
 (segment (start 141.92 110.91) (end 140.84 111.99) (width 0.25) (layer F.Cu) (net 10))
 (segment (start 147.42 110.91) (end 141.92 110.91) (width 0.25) (layer F.Cu) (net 10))
 (segment (start 148.08 103.21) (end 148.08 110.25) (width 0.25) (layer F.Cu) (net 10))
 (segment (start 136.36 97.95) (end 136.36 97.21) (width 0.25) (layer F.Cu) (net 10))
 (segment (start 139.32 100.91) (end 136.36 97.95) (width 0.25) (layer F.Cu) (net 10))
 (segment (start 139.32 104.51) (end 139.32 100.91) (width 0.25) (layer F.Cu) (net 10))
 (segment (start 140.32 105.51) (end 139.32 104.51) (width 0.25) (layer F.Cu) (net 10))
 (segment (start 145.78 105.51) (end 140.32 105.51) (width 0.25) (layer F.Cu) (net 10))
 (segment (start 148.08 103.21) (end 145.78 105.51) (width 0.25) (layer F.Cu) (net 10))
 (segment (start 135.72 99.11) (end 133.82 97.21) (width 0.25) (layer B.Cu) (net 1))
 (segment (start 154.32 99.11) (end 135.72 99.11) (width 0.25) (layer B.Cu) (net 1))
 (segment (start 156.72 101.51) (end 154.32 99.11) (width 0.25) (layer B.Cu) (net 1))
 (segment (start 160.32 101.51) (end 156.72 101.51) (width 0.25) (layer B.Cu) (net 1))
 (segment (start 166.854998 104.81) (end 163.62 104.81) (width 0.25) (layer B.Cu) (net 1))
 (segment (start 169.654998 107.61) (end 166.854998 104.81) (width 0.25) (layer B.Cu) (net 1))
 (segment (start 169.92 107.61) (end 169.654998 107.61) (width 0.25) (layer B.Cu) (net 1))
 (segment (start 163.62 104.81) (end 160.32 101.51) (width 0.25) (layer B.Cu) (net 1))
 (segment (start 169.92 108.21) (end 169.92 107.61) (width 0.25) (layer B.Cu) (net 1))
 (via (at 152.02 110.51) (size 0.8) (drill 0.4) (layers F.Cu B.Cu) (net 5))
 (segment (start 157.98 117.61) (end 159.76 115.83) (width 0.25) (layer F.Cu) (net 5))
 (segment (start 153.85 117.61) (end 157.98 117.61) (width 0.25) (layer F.Cu) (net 5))
 (segment (start 152.02 115.78) (end 153.85 117.61) (width 0.25) (layer F.Cu) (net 5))
 (segment (start 152.02 110.51) (end 152.02 115.78) (width 0.25) (layer F.Cu) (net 5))
 (segment (start 150.2 110.51) (end 152.02 110.51) (width 0.25) (layer B.Cu) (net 5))
 (segment (start 147.99 108.3) (end 150.2 110.51) (width 0.25) (layer B.Cu) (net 5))
 (segment (start 147.99 105.86) (end 147.99 108.3) (width 0.25) (layer B.Cu) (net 5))
 (segment (start 142.04 99.91) (end 147.99 105.86) (width 0.25) (layer B.Cu) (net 5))
 (segment (start 133.98 99.91) (end 142.04 99.91) (width 0.25) (layer B.Cu) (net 5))
 (segment (start 131.28 97.21) (end 133.98 99.91) (width 0.25) (layer B.Cu) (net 5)))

